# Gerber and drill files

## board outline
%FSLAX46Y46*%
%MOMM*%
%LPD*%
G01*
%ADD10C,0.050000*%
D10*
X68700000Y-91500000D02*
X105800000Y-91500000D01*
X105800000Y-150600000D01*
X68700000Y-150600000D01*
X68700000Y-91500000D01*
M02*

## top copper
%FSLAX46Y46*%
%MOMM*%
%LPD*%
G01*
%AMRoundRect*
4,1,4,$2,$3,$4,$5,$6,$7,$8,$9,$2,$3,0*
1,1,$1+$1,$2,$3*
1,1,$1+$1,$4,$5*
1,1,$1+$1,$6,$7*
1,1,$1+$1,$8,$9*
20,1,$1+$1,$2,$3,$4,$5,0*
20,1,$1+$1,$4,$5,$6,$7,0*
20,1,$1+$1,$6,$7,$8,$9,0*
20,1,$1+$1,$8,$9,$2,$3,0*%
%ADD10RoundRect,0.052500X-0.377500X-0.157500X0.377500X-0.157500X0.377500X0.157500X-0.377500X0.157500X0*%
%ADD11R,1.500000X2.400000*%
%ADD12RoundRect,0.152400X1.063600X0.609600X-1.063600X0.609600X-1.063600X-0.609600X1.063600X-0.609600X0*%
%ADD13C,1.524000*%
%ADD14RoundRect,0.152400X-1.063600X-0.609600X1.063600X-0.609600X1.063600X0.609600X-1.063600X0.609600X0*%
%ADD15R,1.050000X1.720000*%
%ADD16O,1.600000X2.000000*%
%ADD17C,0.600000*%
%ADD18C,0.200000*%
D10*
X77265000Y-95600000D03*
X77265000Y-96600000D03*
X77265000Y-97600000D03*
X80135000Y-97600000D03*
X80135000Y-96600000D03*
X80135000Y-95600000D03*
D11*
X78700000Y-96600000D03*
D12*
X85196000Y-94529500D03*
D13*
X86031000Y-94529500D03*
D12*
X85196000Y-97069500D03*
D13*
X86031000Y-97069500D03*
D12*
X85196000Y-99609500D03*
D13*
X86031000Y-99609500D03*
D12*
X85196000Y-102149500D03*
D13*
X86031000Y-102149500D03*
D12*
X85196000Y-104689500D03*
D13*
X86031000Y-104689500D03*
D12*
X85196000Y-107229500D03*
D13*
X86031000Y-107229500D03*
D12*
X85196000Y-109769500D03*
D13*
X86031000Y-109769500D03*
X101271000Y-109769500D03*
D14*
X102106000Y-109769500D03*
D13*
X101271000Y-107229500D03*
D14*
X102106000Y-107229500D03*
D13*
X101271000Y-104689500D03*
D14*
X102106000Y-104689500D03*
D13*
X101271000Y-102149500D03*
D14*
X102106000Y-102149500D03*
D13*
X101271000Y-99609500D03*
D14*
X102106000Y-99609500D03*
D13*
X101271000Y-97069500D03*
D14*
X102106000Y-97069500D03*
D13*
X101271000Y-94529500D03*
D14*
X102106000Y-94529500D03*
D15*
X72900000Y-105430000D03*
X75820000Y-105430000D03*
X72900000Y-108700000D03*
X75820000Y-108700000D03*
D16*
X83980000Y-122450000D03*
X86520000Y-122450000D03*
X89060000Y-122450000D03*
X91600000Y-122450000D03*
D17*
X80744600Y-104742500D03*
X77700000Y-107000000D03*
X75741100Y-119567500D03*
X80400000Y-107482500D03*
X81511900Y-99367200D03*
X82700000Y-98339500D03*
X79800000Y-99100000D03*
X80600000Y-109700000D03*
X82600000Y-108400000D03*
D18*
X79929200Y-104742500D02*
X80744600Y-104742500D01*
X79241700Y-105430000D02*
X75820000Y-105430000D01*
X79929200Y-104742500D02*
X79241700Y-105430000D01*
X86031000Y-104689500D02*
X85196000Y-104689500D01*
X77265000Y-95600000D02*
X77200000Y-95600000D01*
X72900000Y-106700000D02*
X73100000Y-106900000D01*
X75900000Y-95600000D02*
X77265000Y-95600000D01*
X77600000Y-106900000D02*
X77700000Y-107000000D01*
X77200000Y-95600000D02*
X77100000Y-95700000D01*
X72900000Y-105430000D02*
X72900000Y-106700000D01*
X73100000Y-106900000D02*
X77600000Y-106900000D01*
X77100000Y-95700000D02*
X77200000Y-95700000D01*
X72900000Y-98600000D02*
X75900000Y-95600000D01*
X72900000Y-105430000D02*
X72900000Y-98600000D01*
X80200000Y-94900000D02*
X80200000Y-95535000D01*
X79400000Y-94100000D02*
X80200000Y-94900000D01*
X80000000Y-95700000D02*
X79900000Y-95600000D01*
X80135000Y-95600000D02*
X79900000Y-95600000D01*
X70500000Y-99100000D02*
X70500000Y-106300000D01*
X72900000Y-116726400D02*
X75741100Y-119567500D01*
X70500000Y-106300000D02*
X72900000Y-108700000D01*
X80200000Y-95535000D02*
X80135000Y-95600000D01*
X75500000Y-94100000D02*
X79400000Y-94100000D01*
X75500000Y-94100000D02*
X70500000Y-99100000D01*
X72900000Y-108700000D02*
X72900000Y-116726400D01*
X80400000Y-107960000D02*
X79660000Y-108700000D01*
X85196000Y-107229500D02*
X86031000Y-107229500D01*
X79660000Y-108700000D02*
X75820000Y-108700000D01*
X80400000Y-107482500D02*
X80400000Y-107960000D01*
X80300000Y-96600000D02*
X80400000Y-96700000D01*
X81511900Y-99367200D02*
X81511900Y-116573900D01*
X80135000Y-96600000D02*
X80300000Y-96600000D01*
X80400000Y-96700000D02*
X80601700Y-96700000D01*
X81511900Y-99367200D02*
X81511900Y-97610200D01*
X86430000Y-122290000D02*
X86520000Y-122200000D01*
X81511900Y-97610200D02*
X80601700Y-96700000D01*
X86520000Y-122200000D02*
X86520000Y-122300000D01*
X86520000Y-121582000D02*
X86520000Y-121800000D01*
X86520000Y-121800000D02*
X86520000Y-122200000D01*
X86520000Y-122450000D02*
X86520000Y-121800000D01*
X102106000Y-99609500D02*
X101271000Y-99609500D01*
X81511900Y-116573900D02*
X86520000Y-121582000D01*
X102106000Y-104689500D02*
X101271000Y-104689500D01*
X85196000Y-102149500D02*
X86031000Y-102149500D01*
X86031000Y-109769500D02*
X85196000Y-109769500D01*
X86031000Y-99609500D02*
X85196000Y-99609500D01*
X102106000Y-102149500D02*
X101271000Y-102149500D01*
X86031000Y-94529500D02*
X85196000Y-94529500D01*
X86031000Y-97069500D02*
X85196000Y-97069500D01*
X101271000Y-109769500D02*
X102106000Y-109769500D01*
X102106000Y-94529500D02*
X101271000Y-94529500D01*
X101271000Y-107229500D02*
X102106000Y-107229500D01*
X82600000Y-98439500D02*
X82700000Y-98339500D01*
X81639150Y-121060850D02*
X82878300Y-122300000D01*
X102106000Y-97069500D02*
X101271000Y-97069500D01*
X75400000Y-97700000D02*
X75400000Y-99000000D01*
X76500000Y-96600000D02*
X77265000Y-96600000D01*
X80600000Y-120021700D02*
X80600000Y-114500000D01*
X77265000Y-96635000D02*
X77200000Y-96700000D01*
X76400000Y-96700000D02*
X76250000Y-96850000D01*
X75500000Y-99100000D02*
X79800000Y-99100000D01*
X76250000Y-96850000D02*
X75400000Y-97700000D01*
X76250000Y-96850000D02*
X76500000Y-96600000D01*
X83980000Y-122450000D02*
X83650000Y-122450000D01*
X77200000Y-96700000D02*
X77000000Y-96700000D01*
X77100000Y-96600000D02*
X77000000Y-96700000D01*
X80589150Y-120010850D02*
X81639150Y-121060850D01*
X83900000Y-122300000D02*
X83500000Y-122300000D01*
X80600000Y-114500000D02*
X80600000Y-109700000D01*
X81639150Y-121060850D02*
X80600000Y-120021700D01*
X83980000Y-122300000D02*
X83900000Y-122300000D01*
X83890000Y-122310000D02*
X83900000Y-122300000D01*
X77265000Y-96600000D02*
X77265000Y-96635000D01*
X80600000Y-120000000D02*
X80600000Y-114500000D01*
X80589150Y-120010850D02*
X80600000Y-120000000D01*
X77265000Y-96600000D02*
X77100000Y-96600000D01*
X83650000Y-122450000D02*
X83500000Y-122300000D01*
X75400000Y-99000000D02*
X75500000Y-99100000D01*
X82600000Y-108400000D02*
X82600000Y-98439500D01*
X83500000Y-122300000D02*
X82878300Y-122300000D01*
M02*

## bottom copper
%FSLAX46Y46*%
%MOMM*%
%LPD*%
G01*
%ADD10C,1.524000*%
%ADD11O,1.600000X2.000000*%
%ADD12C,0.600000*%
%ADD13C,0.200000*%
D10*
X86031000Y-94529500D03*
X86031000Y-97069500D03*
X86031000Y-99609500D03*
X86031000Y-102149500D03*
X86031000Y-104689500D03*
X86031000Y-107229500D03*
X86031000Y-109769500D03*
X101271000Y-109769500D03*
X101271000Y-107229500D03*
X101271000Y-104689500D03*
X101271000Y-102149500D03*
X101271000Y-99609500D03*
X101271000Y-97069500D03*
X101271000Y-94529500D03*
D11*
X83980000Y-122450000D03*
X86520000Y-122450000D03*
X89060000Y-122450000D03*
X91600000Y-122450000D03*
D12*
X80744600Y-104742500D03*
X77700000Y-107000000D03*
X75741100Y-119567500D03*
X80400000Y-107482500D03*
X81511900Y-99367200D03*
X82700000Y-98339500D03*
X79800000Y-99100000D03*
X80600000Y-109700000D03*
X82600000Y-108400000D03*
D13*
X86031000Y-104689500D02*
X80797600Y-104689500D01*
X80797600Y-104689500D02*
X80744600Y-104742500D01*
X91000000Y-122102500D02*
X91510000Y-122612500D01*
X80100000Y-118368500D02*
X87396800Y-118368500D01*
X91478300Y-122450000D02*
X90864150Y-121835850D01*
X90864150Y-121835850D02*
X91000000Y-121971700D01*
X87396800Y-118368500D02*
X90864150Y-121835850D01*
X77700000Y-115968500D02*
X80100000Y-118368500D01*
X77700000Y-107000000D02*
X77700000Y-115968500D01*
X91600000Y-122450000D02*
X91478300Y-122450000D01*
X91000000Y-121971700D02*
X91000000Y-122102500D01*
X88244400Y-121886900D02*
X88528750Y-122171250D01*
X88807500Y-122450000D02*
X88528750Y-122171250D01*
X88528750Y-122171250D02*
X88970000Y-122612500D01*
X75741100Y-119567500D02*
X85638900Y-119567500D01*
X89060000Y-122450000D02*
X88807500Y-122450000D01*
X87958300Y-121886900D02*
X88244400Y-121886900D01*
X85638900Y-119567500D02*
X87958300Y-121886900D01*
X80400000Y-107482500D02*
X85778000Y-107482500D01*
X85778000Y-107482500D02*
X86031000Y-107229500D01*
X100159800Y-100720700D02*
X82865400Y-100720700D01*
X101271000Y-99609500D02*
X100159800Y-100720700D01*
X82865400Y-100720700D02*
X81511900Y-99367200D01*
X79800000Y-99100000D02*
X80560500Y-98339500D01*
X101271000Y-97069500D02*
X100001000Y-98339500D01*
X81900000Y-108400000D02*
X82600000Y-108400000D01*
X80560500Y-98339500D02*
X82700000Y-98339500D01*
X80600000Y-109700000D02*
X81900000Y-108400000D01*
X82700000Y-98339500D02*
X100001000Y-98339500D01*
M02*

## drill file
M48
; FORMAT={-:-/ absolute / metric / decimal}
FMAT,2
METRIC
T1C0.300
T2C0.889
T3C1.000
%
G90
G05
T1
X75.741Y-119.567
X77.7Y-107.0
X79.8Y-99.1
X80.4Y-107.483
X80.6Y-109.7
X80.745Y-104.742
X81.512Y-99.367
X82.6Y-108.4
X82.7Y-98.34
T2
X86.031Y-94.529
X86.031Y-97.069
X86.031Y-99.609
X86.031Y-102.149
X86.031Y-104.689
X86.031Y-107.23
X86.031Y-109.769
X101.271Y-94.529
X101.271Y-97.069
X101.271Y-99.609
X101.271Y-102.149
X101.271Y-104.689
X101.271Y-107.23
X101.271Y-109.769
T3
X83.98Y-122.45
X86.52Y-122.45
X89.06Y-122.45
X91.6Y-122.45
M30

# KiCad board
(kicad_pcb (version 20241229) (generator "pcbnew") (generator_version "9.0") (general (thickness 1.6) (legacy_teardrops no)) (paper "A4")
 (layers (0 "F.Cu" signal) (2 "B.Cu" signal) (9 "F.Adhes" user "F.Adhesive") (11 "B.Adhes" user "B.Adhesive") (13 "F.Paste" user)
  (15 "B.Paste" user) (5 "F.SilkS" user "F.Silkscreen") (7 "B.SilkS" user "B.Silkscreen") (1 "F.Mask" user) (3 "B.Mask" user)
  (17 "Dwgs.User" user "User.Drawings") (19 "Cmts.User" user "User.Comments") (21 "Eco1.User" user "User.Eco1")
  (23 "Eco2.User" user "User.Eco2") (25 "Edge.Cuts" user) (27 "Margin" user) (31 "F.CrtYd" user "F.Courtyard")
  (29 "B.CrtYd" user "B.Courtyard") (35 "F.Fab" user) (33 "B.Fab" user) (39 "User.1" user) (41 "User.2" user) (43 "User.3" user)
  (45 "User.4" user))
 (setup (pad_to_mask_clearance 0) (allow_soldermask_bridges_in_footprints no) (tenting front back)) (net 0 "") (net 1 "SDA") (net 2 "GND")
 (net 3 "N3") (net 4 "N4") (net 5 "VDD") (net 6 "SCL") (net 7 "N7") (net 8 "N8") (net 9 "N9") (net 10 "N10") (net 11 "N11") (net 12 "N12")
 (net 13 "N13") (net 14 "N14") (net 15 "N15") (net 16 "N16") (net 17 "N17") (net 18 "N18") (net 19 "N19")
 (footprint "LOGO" (layer "F.Cu") (at 72.1 95)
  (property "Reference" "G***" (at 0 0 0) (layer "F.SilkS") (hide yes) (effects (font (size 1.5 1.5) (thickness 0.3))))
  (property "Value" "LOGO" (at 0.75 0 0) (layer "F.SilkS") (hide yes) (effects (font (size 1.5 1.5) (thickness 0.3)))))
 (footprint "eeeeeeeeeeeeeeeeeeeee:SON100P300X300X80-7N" (layer "F.Cu") (at 78.7 96.6)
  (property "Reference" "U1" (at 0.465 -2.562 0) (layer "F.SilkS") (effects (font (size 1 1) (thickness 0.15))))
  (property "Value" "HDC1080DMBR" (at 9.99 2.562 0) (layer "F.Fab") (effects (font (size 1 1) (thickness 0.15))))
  (pad "1" smd roundrect (at -1.435 -1) (size 0.86 0.42) (layers "F.Cu" "F.Mask" "F.Paste") (roundrect_rratio 0.125) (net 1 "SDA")
   (solder_mask_margin 0.102))
  (pad "2" smd roundrect (at -1.435 0) (size 0.86 0.42) (layers "F.Cu" "F.Mask" "F.Paste") (roundrect_rratio 0.125) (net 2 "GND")
   (solder_mask_margin 0.102))
  (pad "3" smd roundrect (at -1.435 1) (size 0.86 0.42) (layers "F.Cu" "F.Mask" "F.Paste") (roundrect_rratio 0.125) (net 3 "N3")
   (solder_mask_margin 0.102))
  (pad "4" smd roundrect (at 1.435 1) (size 0.86 0.42) (layers "F.Cu" "F.Mask" "F.Paste") (roundrect_rratio 0.125) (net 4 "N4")
   (solder_mask_margin 0.102))
  (pad "5" smd roundrect (at 1.435 0) (size 0.86 0.42) (layers "F.Cu" "F.Mask" "F.Paste") (roundrect_rratio 0.125) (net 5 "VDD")
   (solder_mask_margin 0.102))
  (pad "6" smd roundrect (at 1.435 -1) (size 0.86 0.42) (layers "F.Cu" "F.Mask" "F.Paste") (roundrect_rratio 0.125) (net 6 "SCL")
   (solder_mask_margin 0.102))
  (pad "7" smd rect (at 0 0) (size 1.5 2.4) (layers "F.Cu" "F.Mask") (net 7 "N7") (solder_mask_margin 0.102)))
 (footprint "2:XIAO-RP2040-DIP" (layer "F.Cu") (at 93.651 102.1495)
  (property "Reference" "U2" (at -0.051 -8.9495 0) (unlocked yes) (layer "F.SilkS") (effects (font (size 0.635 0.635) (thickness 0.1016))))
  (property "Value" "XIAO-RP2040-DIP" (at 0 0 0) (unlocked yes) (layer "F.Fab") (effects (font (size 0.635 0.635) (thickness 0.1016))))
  (pad "1" smd roundrect (at -8.455 -7.62 180) (size 2.432 1.524) (layers "F.Cu" "F.Mask") (roundrect_rratio 0.1) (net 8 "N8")
   (thermal_bridge_angle 45))
  (pad "1" thru_hole circle (at -7.62 -7.62 180) (size 1.524 1.524) (drill 0.889) (layers "*.Cu" "*.Mask") (remove_unused_layers no)
   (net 8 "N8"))
  (pad "2" smd roundrect (at -8.455 -5.08 180) (size 2.432 1.524) (layers "F.Cu" "F.Mask") (roundrect_rratio 0.1) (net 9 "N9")
   (thermal_bridge_angle 45))
  (pad "2" thru_hole circle (at -7.62 -5.08 180) (size 1.524 1.524) (drill 0.889) (layers "*.Cu" "*.Mask") (remove_unused_layers no)
   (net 9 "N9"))
  (pad "3" smd roundrect (at -8.455 -2.54 180) (size 2.432 1.524) (layers "F.Cu" "F.Mask") (roundrect_rratio 0.1) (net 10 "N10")
   (thermal_bridge_angle 45))
  (pad "3" thru_hole circle (at -7.62 -2.54 180) (size 1.524 1.524) (drill 0.889) (layers "*.Cu" "*.Mask") (remove_unused_layers no)
   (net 10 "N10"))
  (pad "4" smd roundrect (at -8.455 0 180) (size 2.432 1.524) (layers "F.Cu" "F.Mask") (roundrect_rratio 0.1) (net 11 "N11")
   (thermal_bridge_angle 45))
  (pad "4" thru_hole circle (at -7.62 0 180) (size 1.524 1.524) (drill 0.889) (layers "*.Cu" "*.Mask") (remove_unused_layers no)
   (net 11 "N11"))
  (pad "5" smd roundrect (at -8.455 2.54 180) (size 2.432 1.524) (layers "F.Cu" "F.Mask") (roundrect_rratio 0.1) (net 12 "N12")
   (thermal_bridge_angle 45))
  (pad "5" thru_hole circle (at -7.62 2.54 180) (size 1.524 1.524) (drill 0.889) (layers "*.Cu" "*.Mask") (remove_unused_layers no)
   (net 12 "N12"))
  (pad "6" smd roundrect (at -8.455 5.08 180) (size 2.432 1.524) (layers "F.Cu" "F.Mask") (roundrect_rratio 0.1) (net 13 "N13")
   (thermal_bridge_angle 45))
  (pad "6" thru_hole circle (at -7.62 5.08 180) (size 1.524 1.524) (drill 0.889) (layers "*.Cu" "*.Mask") (remove_unused_layers no)
   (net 13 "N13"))
  (pad "7" smd roundrect (at -8.455 7.62 180) (size 2.432 1.524) (layers "F.Cu" "F.Mask") (roundrect_rratio 0.1) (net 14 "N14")
   (thermal_bridge_angle 45))
  (pad "7" thru_hole circle (at -7.62 7.62 180) (size 1.524 1.524) (drill 0.889) (layers "*.Cu" "*.Mask") (remove_unused_layers no)
   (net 14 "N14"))
  (pad "8" thru_hole circle (at 7.62 7.62) (size 1.524 1.524) (drill 0.889) (layers "*.Cu" "*.Mask") (remove_unused_layers no)
   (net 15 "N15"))
  (pad "8" smd roundrect (at 8.455 7.62) (size 2.432 1.524) (layers "F.Cu" "F.Mask") (roundrect_rratio 0.1) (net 15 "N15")
   (thermal_bridge_angle 45))
  (pad "9" thru_hole circle (at 7.62 5.08) (size 1.524 1.524) (drill 0.889) (layers "*.Cu" "*.Mask") (remove_unused_layers no)
   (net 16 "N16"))
  (pad "9" smd roundrect (at 8.455 5.08) (size 2.432 1.524) (layers "F.Cu" "F.Mask") (roundrect_rratio 0.1) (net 16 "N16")
   (thermal_bridge_angle 45))
  (pad "10" thru_hole circle (at 7.62 2.54) (size 1.524 1.524) (drill 0.889) (layers "*.Cu" "*.Mask") (remove_unused_layers no)
   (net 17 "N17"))
  (pad "10" smd roundrect (at 8.455 2.54) (size 2.432 1.524) (layers "F.Cu" "F.Mask") (roundrect_rratio 0.1) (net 17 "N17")
   (thermal_bridge_angle 45))
  (pad "11" thru_hole circle (at 7.62 0) (size 1.524 1.524) (drill 0.889) (layers "*.Cu" "*.Mask") (remove_unused_layers no) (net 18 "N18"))
  (pad "11" smd roundrect (at 8.455 0) (size 2.432 1.524) (layers "F.Cu" "F.Mask") (roundrect_rratio 0.1) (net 18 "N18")
   (thermal_bridge_angle 45))
  (pad "12" thru_hole circle (at 7.62 -2.54) (size 1.524 1.524) (drill 0.889) (layers "*.Cu" "*.Mask") (remove_unused_layers no)
   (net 5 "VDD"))
  (pad "12" smd roundrect (at 8.455 -2.54) (size 2.432 1.524) (layers "F.Cu" "F.Mask") (roundrect_rratio 0.1) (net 5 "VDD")
   (thermal_bridge_angle 45))
  (pad "13" thru_hole circle (at 7.62 -5.08) (size 1.524 1.524) (drill 0.889) (layers "*.Cu" "*.Mask") (remove_unused_layers no)
   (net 2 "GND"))
  (pad "13" smd roundrect (at 8.455 -5.08) (size 2.432 1.524) (layers "F.Cu" "F.Mask") (roundrect_rratio 0.1) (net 2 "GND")
   (thermal_bridge_angle 45))
  (pad "14" thru_hole circle (at 7.62 -7.62) (size 1.524 1.524) (drill 0.889) (layers "*.Cu" "*.Mask") (remove_unused_layers no)
   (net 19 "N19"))
  (pad "14" smd roundrect (at 8.455 -7.62) (size 2.432 1.524) (layers "F.Cu" "F.Mask") (roundrect_rratio 0.1) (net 19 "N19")
   (thermal_bridge_angle 45)))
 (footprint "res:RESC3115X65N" (layer "F.Cu") (at 74.36 105.43)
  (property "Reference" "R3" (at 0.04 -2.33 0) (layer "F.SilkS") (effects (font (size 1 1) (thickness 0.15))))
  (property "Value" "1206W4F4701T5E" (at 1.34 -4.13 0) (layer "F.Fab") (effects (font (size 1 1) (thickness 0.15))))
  (pad "1" smd rect (at -1.46 0) (size 1.05 1.72) (layers "F.Cu" "F.Mask" "F.Paste") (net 1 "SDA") (solder_mask_margin 0.102))
  (pad "2" smd rect (at 1.46 0) (size 1.05 1.72) (layers "F.Cu" "F.Mask" "F.Paste") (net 12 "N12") (solder_mask_margin 0.102)))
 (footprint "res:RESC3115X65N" (layer "F.Cu") (at 74.36 108.7)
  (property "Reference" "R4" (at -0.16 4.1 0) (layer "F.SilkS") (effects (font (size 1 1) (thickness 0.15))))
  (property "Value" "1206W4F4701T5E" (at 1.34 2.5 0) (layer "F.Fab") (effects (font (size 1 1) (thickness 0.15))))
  (pad "1" smd rect (at -1.46 0) (size 1.05 1.72) (layers "F.Cu" "F.Mask" "F.Paste") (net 6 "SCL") (solder_mask_margin 0.102))
  (pad "2" smd rect (at 1.46 0) (size 1.05 1.72) (layers "F.Cu" "F.Mask" "F.Paste") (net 13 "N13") (solder_mask_margin 0.102)))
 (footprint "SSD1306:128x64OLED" (layer "F.Cu") (at 87.6 133.05)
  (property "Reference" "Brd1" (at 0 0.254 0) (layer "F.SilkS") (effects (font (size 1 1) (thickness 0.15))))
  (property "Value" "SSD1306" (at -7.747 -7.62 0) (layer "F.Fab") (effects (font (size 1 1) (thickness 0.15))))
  (pad "1" thru_hole oval (at -3.62 -10.6 90) (size 2 1.6) (drill 1) (layers "*.Cu" "*.Mask") (remove_unused_layers no) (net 2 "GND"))
  (pad "2" thru_hole oval (at -1.08 -10.6 90) (size 2 1.6) (drill 1) (layers "*.Cu" "*.Mask") (remove_unused_layers no) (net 5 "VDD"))
  (pad "3" thru_hole oval (at 1.46 -10.6 90) (size 2 1.6) (drill 1) (layers "*.Cu" "*.Mask") (remove_unused_layers no) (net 6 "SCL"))
  (pad "4" thru_hole oval (at 4 -10.6 90) (size 2 1.6) (drill 1) (layers "*.Cu" "*.Mask") (remove_unused_layers no) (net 1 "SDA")))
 (gr_rect (start 68.7 91.5) (end 105.8 150.6) (stroke (width 0.05) (type default)) (fill no) (layer "Edge.Cuts"))
 (segment (start 79.9292 104.7425) (end 80.7446 104.7425) (width 0.2) (layer "F.Cu") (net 12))
 (segment (start 79.2417 105.43) (end 75.82 105.43) (width 0.2) (layer "F.Cu") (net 12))
 (segment (start 79.9292 104.7425) (end 79.2417 105.43) (width 0.2) (layer "F.Cu") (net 12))
 (segment (start 86.031 104.6895) (end 85.196 104.6895) (width 0.2) (layer "F.Cu") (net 12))
 (via (at 80.7446 104.7425) (size 0.6) (drill 0.3) (layers "F.Cu" "B.Cu") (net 12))
 (segment (start 86.031 104.6895) (end 80.7976 104.6895) (width 0.2) (layer "B.Cu") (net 12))
 (segment (start 80.7976 104.6895) (end 80.7446 104.7425) (width 0.2) (layer "B.Cu") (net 12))
 (segment (start 77.265 95.6) (end 77.2 95.6) (width 0.2) (layer "F.Cu") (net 1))
 (segment (start 72.9 106.7) (end 73.1 106.9) (width 0.2) (layer "F.Cu") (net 1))
 (segment (start 75.9 95.6) (end 77.265 95.6) (width 0.2) (layer "F.Cu") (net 1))
 (segment (start 77.6 106.9) (end 77.7 107) (width 0.2) (layer "F.Cu") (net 1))
 (segment (start 77.2 95.6) (end 77.1 95.7) (width 0.2) (layer "F.Cu") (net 1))
 (segment (start 72.9 105.43) (end 72.9 106.7) (width 0.2) (layer "F.Cu") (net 1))
 (segment (start 73.1 106.9) (end 77.6 106.9) (width 0.2) (layer "F.Cu") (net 1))
 (segment (start 77.1 95.7) (end 77.2 95.7) (width 0.2) (layer "F.Cu") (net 1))
 (segment (start 72.9 98.6) (end 75.9 95.6) (width 0.2) (layer "F.Cu") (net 1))
 (segment (start 72.9 105.43) (end 72.9 98.6) (width 0.2) (layer "F.Cu") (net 1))
 (via (at 77.7 107) (size 0.6) (drill 0.3) (layers "F.Cu" "B.Cu") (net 1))
 (segment (start 91 122.1025) (end 91.51 122.6125) (width 0.2) (layer "B.Cu") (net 1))
 (segment (start 80.1 118.3685) (end 87.3968 118.3685) (width 0.2) (layer "B.Cu") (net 1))
 (segment (start 91.4783 122.45) (end 90.86415 121.83585) (width 0.2) (layer "B.Cu") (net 1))
 (segment (start 90.86415 121.83585) (end 91 121.9717) (width 0.2) (layer "B.Cu") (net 1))
 (segment (start 87.3968 118.3685) (end 90.86415 121.83585) (width 0.2) (layer "B.Cu") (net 1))
 (segment (start 77.7 115.9685) (end 80.1 118.3685) (width 0.2) (layer "B.Cu") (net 1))
 (segment (start 77.7 107) (end 77.7 115.9685) (width 0.2) (layer "B.Cu") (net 1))
 (segment (start 91.6 122.45) (end 91.4783 122.45) (width 0.2) (layer "B.Cu") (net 1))
 (segment (start 91 121.9717) (end 91 122.1025) (width 0.2) (layer "B.Cu") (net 1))
 (segment (start 80.2 94.9) (end 80.2 95.535) (width 0.2) (layer "F.Cu") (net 6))
 (segment (start 79.4 94.1) (end 80.2 94.9) (width 0.2) (layer "F.Cu") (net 6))
 (segment (start 80 95.7) (end 79.9 95.6) (width 0.2) (layer "F.Cu") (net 6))
 (segment (start 80.135 95.6) (end 79.9 95.6) (width 0.2) (layer "F.Cu") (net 6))
 (segment (start 70.5 99.1) (end 70.5 106.3) (width 0.2) (layer "F.Cu") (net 6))
 (segment (start 72.9 116.7264) (end 75.7411 119.5675) (width 0.2) (layer "F.Cu") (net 6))
 (segment (start 70.5 106.3) (end 72.9 108.7) (width 0.2) (layer "F.Cu") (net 6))
 (segment (start 80.2 95.535) (end 80.135 95.6) (width 0.2) (layer "F.Cu") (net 6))
 (segment (start 75.5 94.1) (end 79.4 94.1) (width 0.2) (layer "F.Cu") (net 6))
 (segment (start 75.5 94.1) (end 70.5 99.1) (width 0.2) (layer "F.Cu") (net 6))
 (segment (start 72.9 108.7) (end 72.9 116.7264) (width 0.2) (layer "F.Cu") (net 6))
 (via (at 75.7411 119.5675) (size 0.6) (drill 0.3) (layers "F.Cu" "B.Cu") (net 6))
 (segment (start 88.2444 121.8869) (end 88.52875 122.17125) (width 0.2) (layer "B.Cu") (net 6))
 (segment (start 88.8075 122.45) (end 88.52875 122.17125) (width 0.2) (layer "B.Cu") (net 6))
 (segment (start 88.52875 122.17125) (end 88.97 122.6125) (width 0.2) (layer "B.Cu") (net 6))
 (segment (start 75.7411 119.5675) (end 85.6389 119.5675) (width 0.2) (layer "B.Cu") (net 6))
 (segment (start 89.06 122.45) (end 88.8075 122.45) (width 0.2) (layer "B.Cu") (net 6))
 (segment (start 87.9583 121.8869) (end 88.2444 121.8869) (width 0.2) (layer "B.Cu") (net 6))
 (segment (start 85.6389 119.5675) (end 87.9583 121.8869) (width 0.2) (layer "B.Cu") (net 6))
 (segment (start 80.4 107.96) (end 79.66 108.7) (width 0.2) (layer "F.Cu") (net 13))
 (segment (start 85.196 107.2295) (end 86.031 107.2295) (width 0.2) (layer "F.Cu") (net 13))
 (segment (start 79.66 108.7) (end 75.82 108.7) (width 0.2) (layer "F.Cu") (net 13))
 (segment (start 80.4 107.4825) (end 80.4 107.96) (width 0.2) (layer "F.Cu") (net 13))
 (via (at 80.4 107.4825) (size 0.6) (drill 0.3) (layers "F.Cu" "B.Cu") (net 13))
 (segment (start 80.4 107.4825) (end 85.778 107.4825) (width 0.2) (layer "B.Cu") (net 13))
 (segment (start 85.778 107.4825) (end 86.031 107.2295) (width 0.2) (layer "B.Cu") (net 13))
 (segment (start 80.3 96.6) (end 80.4 96.7) (width 0.2) (layer "F.Cu") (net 5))
 (segment (start 81.5119 99.3672) (end 81.5119 116.5739) (width 0.2) (layer "F.Cu") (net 5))
 (segment (start 80.135 96.6) (end 80.3 96.6) (width 0.2) (layer "F.Cu") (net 5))
 (segment (start 80.4 96.7) (end 80.6017 96.7) (width 0.2) (layer "F.Cu") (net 5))
 (segment (start 81.5119 99.3672) (end 81.5119 97.6102) (width 0.2) (layer "F.Cu") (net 5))
 (segment (start 86.43 122.29) (end 86.52 122.2) (width 0.2) (layer "F.Cu") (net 5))
 (segment (start 81.5119 97.6102) (end 80.6017 96.7) (width 0.2) (layer "F.Cu") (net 5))
 (segment (start 86.52 122.2) (end 86.52 122.3) (width 0.2) (layer "F.Cu") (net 5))
 (segment (start 86.52 121.582) (end 86.52 121.8) (width 0.2) (layer "F.Cu") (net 5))
 (segment (start 86.52 121.8) (end 86.52 122.2) (width 0.2) (layer "F.Cu") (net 5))
 (segment (start 86.52 122.45) (end 86.52 121.8) (width 0.2) (layer "F.Cu") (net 5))
 (segment (start 102.106 99.6095) (end 101.271 99.6095) (width 0.2) (layer "F.Cu") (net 5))
 (segment (start 81.5119 116.5739) (end 86.52 121.582) (width 0.2) (layer "F.Cu") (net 5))
 (via (at 81.5119 99.3672) (size 0.6) (drill 0.3) (layers "F.Cu" "B.Cu") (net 5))
 (segment (start 100.1598 100.7207) (end 82.8654 100.7207) (width 0.2) (layer "B.Cu") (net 5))
 (segment (start 101.271 99.6095) (end 100.1598 100.7207) (width 0.2) (layer "B.Cu") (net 5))
 (segment (start 82.8654 100.7207) (end 81.5119 99.3672) (width 0.2) (layer "B.Cu") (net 5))
 (segment (start 102.106 104.6895) (end 101.271 104.6895) (width 0.2) (layer "F.Cu") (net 17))
 (segment (start 85.196 102.1495) (end 86.031 102.1495) (width 0.2) (layer "F.Cu") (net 11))
 (segment (start 86.031 109.7695) (end 85.196 109.7695) (width 0.2) (layer "F.Cu") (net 14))
 (segment (start 86.031 99.6095) (end 85.196 99.6095) (width 0.2) (layer "F.Cu") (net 10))
 (segment (start 102.106 102.1495) (end 101.271 102.1495) (width 0.2) (layer "F.Cu") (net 18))
 (segment (start 86.031 94.5295) (end 85.196 94.5295) (width 0.2) (layer "F.Cu") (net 8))
 (segment (start 86.031 97.0695) (end 85.196 97.0695) (width 0.2) (layer "F.Cu") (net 9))
 (segment (start 101.271 109.7695) (end 102.106 109.7695) (width 0.2) (layer "F.Cu") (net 15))
 (segment (start 102.106 94.5295) (end 101.271 94.5295) (width 0.2) (layer "F.Cu") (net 19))
 (segment (start 101.271 107.2295) (end 102.106 107.2295) (width 0.2) (layer "F.Cu") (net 16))
 (segment (start 82.6 98.4395) (end 82.7 98.3395) (width 0.2) (layer "F.Cu") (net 2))
 (segment (start 81.63915 121.06085) (end 82.8783 122.3) (width 0.2) (layer "F.Cu") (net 2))
 (segment (start 102.106 97.0695) (end 101.271 97.0695) (width 0.2) (layer "F.Cu") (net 2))
 (segment (start 75.4 97.7) (end 75.4 99) (width 0.2) (layer "F.Cu") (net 2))
 (segment (start 76.5 96.6) (end 77.265 96.6) (width 0.2) (layer "F.Cu") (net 2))
 (segment (start 80.6 120.0217) (end 80.6 114.5) (width 0.2) (layer "F.Cu") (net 2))
 (segment (start 77.265 96.635) (end 77.2 96.7) (width 0.2) (layer "F.Cu") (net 2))
 (segment (start 76.4 96.7) (end 76.25 96.85) (width 0.2) (layer "F.Cu") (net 2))
 (segment (start 75.5 99.1) (end 79.8 99.1) (width 0.2) (layer "F.Cu") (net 2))
 (segment (start 76.25 96.85) (end 75.4 97.7) (width 0.2) (layer "F.Cu") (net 2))
 (segment (start 76.25 96.85) (end 76.5 96.6) (width 0.2) (layer "F.Cu") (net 2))
 (segment (start 83.98 122.45) (end 83.65 122.45) (width 0.2) (layer "F.Cu") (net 2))
 (segment (start 77.2 96.7) (end 77 96.7) (width 0.2) (layer "F.Cu") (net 2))
 (segment (start 77.1 96.6) (end 77 96.7) (width 0.2) (layer "F.Cu") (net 2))
 (segment (start 80.58915 120.01085) (end 81.63915 121.06085) (width 0.2) (layer "F.Cu") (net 2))
 (segment (start 83.9 122.3) (end 83.5 122.3) (width 0.2) (layer "F.Cu") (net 2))
 (segment (start 80.6 114.5) (end 80.6 109.7) (width 0.2) (layer "F.Cu") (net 2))
 (segment (start 81.63915 121.06085) (end 80.6 120.0217) (width 0.2) (layer "F.Cu") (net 2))
 (segment (start 83.98 122.3) (end 83.9 122.3) (width 0.2) (layer "F.Cu") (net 2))
 (segment (start 83.89 122.31) (end 83.9 122.3) (width 0.2) (layer "F.Cu") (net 2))
 (segment (start 77.265 96.6) (end 77.265 96.635) (width 0.2) (layer "F.Cu") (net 2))
 (segment (start 80.6 120) (end 80.6 114.5) (width 0.2) (layer "F.Cu") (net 2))
 (segment (start 80.58915 120.01085) (end 80.6 120) (width 0.2) (layer "F.Cu") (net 2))
 (segment (start 77.265 96.6) (end 77.1 96.6) (width 0.2) (layer "F.Cu") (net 2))
 (segment (start 83.65 122.45) (end 83.5 122.3) (width 0.2) (layer "F.Cu") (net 2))
 (segment (start 75.4 99) (end 75.5 99.1) (width 0.2) (layer "F.Cu") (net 2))
 (segment (start 82.6 108.4) (end 82.6 98.4395) (width 0.2) (layer "F.Cu") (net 2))
 (segment (start 83.5 122.3) (end 82.8783 122.3) (width 0.2) (layer "F.Cu") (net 2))
 (via (at 82.7 98.3395) (size 0.6) (drill 0.3) (layers "F.Cu" "B.Cu") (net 2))
 (via (at 79.8 99.1) (size 0.6) (drill 0.3) (layers "F.Cu" "B.Cu") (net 2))
 (via (at 80.6 109.7) (size 0.6) (drill 0.3) (layers "F.Cu" "B.Cu") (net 2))
 (via (at 82.6 108.4) (size 0.6) (drill 0.3) (layers "F.Cu" "B.Cu") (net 2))
 (segment (start 79.8 99.1) (end 80.5605 98.3395) (width 0.2) (layer "B.Cu") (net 2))
 (segment (start 101.271 97.0695) (end 100.001 98.3395) (width 0.2) (layer "B.Cu") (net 2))
 (segment (start 81.9 108.4) (end 82.6 108.4) (width 0.2) (layer "B.Cu") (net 2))
 (segment (start 80.5605 98.3395) (end 82.7 98.3395) (width 0.2) (layer "B.Cu") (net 2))
 (segment (start 80.6 109.7) (end 81.9 108.4) (width 0.2) (layer "B.Cu") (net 2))
 (segment (start 82.7 98.3395) (end 100.001 98.3395) (width 0.2) (layer "B.Cu") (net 2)))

